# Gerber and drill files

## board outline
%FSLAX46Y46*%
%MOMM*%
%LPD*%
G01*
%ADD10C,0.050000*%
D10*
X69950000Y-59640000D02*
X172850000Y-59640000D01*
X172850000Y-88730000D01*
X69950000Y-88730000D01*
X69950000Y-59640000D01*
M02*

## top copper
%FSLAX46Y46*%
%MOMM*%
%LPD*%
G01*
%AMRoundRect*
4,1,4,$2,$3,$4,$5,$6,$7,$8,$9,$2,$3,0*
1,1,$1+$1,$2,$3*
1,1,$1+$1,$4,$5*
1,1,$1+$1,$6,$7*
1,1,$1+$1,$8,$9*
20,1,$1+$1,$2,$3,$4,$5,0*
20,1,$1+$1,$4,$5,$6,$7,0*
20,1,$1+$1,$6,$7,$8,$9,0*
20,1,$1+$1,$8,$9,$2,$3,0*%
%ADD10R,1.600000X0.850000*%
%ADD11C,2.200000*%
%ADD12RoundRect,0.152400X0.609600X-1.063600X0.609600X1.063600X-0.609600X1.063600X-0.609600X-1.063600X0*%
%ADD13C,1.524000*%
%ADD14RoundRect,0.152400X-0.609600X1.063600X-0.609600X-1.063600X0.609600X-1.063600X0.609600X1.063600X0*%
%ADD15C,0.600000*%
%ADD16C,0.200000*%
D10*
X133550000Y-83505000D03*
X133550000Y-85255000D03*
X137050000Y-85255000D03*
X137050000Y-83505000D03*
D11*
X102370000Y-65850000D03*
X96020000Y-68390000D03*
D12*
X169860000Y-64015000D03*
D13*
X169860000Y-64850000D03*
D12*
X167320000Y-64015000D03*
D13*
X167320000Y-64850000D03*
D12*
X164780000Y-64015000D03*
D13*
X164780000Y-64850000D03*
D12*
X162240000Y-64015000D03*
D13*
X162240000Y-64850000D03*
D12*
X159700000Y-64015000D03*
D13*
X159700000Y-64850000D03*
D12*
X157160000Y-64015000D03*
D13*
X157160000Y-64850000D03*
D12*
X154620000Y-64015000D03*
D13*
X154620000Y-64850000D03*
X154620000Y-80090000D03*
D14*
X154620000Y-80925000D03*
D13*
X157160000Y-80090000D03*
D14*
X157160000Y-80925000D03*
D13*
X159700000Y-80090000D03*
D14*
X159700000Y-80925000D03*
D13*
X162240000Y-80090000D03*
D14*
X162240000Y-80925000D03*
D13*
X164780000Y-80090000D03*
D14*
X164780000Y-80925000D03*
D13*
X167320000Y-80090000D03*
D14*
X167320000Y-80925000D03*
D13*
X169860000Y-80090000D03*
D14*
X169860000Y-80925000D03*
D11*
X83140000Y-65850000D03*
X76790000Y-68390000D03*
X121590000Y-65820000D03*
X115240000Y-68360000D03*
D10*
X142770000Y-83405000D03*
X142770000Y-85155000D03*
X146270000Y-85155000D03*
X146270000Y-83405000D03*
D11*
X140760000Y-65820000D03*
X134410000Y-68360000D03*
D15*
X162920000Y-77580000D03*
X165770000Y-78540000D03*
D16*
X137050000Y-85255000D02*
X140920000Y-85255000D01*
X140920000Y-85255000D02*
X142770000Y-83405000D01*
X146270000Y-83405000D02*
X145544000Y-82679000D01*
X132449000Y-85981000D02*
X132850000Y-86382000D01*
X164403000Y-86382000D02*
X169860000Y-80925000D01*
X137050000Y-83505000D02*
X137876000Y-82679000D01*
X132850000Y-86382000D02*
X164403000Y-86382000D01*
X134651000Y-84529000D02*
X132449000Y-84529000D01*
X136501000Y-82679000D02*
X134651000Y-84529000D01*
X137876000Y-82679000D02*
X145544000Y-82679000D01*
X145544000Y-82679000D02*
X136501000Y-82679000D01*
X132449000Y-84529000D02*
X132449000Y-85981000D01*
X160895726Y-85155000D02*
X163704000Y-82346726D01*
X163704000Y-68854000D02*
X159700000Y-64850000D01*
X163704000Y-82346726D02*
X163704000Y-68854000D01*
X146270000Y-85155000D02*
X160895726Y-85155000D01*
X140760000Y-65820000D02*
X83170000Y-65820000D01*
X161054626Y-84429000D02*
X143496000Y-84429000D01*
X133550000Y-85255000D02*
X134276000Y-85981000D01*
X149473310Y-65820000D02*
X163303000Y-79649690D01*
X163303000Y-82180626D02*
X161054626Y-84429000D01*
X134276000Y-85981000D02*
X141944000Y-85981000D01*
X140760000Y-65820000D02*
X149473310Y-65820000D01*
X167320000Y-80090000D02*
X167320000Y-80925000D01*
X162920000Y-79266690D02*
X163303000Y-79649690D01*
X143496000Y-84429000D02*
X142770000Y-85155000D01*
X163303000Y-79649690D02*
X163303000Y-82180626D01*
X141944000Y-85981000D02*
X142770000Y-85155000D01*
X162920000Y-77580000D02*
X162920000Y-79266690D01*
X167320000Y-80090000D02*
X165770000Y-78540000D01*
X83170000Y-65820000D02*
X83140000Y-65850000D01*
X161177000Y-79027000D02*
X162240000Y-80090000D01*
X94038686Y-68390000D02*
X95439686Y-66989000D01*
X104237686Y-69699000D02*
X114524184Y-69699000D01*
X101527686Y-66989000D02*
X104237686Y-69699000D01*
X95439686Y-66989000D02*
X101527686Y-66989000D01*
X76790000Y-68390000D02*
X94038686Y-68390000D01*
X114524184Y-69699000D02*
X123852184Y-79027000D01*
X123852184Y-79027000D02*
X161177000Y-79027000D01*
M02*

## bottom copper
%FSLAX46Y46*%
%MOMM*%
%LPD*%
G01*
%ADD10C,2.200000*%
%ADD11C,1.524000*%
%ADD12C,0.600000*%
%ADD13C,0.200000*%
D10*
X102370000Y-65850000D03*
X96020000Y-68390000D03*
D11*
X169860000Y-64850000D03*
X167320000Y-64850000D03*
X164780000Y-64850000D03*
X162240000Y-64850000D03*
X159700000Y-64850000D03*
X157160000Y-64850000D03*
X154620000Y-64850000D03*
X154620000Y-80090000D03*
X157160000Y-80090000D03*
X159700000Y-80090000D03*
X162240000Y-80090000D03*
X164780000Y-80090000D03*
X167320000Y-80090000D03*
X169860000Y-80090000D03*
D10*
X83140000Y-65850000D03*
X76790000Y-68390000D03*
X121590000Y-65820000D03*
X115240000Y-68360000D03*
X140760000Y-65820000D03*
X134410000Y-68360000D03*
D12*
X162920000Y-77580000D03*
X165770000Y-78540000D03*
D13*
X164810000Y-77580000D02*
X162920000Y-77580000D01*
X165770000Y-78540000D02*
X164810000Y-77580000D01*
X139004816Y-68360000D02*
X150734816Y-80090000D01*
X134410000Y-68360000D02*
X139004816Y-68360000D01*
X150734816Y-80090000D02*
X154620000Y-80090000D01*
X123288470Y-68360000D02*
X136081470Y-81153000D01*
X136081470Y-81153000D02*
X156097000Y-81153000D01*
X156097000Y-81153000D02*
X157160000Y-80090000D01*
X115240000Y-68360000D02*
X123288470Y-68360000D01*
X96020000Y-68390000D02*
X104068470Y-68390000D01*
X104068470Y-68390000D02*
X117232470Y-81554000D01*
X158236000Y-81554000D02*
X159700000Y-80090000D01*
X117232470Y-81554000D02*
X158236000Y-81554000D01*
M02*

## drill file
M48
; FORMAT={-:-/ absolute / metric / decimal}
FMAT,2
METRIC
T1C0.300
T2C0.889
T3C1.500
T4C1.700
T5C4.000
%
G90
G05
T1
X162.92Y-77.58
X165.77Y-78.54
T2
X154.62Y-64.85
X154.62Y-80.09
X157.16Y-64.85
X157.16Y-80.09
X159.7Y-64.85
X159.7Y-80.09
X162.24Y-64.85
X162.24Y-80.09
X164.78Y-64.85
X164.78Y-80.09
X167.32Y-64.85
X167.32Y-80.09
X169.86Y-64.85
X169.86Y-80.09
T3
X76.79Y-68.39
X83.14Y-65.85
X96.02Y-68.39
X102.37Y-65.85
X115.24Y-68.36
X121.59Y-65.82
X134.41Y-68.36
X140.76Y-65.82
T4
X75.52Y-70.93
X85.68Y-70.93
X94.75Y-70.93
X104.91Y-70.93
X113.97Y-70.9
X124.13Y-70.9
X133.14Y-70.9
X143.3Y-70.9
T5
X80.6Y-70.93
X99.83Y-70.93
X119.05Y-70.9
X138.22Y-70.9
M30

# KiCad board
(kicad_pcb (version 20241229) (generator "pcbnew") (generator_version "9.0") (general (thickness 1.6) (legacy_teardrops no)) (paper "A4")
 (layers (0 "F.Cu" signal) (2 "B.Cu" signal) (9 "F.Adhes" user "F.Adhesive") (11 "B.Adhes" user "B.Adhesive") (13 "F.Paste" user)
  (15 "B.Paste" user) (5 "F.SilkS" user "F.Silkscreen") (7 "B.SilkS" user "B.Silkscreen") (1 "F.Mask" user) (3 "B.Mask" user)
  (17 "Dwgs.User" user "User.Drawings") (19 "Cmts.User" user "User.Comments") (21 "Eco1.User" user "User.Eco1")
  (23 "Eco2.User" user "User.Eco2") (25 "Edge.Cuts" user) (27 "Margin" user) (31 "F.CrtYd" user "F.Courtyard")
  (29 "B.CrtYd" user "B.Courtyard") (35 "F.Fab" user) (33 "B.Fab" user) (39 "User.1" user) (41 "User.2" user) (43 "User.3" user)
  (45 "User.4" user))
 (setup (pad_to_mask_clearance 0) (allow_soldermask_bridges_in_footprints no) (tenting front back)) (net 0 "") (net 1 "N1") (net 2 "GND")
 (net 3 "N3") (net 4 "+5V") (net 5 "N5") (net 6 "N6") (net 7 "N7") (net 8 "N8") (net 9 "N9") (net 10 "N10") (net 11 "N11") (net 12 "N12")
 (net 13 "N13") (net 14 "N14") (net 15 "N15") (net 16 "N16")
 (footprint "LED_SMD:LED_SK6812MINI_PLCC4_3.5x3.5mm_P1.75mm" (layer "F.Cu") (at 135.3 84.38)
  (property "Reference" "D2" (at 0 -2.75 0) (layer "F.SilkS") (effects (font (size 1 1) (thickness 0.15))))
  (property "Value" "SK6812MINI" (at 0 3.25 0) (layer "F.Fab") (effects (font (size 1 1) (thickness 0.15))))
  (pad "1" smd rect (at -1.75 -0.875) (size 1.6 0.85) (layers "F.Cu" "F.Mask" "F.Paste") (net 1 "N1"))
  (pad "2" smd rect (at -1.75 0.875) (size 1.6 0.85) (layers "F.Cu" "F.Mask" "F.Paste") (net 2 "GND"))
  (pad "3" smd rect (at 1.75 0.875) (size 1.6 0.85) (layers "F.Cu" "F.Mask" "F.Paste") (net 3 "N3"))
  (pad "4" smd rect (at 1.75 -0.875) (size 1.6 0.85) (layers "F.Cu" "F.Mask" "F.Paste") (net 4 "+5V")))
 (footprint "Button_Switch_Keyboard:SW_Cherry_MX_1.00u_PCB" (layer "F.Cu") (at 102.37 65.85)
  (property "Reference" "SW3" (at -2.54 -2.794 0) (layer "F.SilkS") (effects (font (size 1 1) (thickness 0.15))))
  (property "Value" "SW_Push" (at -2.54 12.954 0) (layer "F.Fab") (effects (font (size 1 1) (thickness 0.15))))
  (pad "" np_thru_hole circle (at -7.62 5.08) (size 1.7 1.7) (drill 1.7) (layers "*.Cu" "*.Mask"))
  (pad "" np_thru_hole circle (at -2.54 5.08) (size 4 4) (drill 4) (layers "*.Cu" "*.Mask"))
  (pad "" np_thru_hole circle (at 2.54 5.08) (size 1.7 1.7) (drill 1.7) (layers "*.Cu" "*.Mask"))
  (pad "1" thru_hole circle (at 0 0) (size 2.2 2.2) (drill 1.5) (layers "*.Cu" "*.Mask") (remove_unused_layers no) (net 2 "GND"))
  (pad "2" thru_hole circle (at -6.35 2.54) (size 2.2 2.2) (drill 1.5) (layers "*.Cu" "*.Mask") (remove_unused_layers no) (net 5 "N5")))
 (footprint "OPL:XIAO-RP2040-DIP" (layer "F.Cu") (at 162.24 72.47 -90)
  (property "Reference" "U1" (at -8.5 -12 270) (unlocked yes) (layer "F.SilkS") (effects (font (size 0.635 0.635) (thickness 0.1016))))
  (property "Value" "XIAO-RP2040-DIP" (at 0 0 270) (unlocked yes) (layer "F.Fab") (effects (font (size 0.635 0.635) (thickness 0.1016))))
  (pad "1" smd roundrect (at -8.455 -7.62 90) (size 2.432 1.524) (layers "F.Cu" "F.Mask") (roundrect_rratio 0.1) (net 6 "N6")
   (thermal_bridge_angle 45))
  (pad "1" thru_hole circle (at -7.62 -7.62 90) (size 1.524 1.524) (drill 0.889) (layers "*.Cu" "*.Mask") (remove_unused_layers no)
   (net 6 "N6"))
  (pad "2" smd roundrect (at -8.455 -5.08 90) (size 2.432 1.524) (layers "F.Cu" "F.Mask") (roundrect_rratio 0.1) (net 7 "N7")
   (thermal_bridge_angle 45))
  (pad "2" thru_hole circle (at -7.62 -5.08 90) (size 1.524 1.524) (drill 0.889) (layers "*.Cu" "*.Mask") (remove_unused_layers no)
   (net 7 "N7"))
  (pad "3" smd roundrect (at -8.455 -2.54 90) (size 2.432 1.524) (layers "F.Cu" "F.Mask") (roundrect_rratio 0.1) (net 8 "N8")
   (thermal_bridge_angle 45))
  (pad "3" thru_hole circle (at -7.62 -2.54 90) (size 1.524 1.524) (drill 0.889) (layers "*.Cu" "*.Mask") (remove_unused_layers no)
   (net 8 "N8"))
  (pad "4" smd roundrect (at -8.455 0 90) (size 2.432 1.524) (layers "F.Cu" "F.Mask") (roundrect_rratio 0.1) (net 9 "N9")
   (thermal_bridge_angle 45))
  (pad "4" thru_hole circle (at -7.62 0 90) (size 1.524 1.524) (drill 0.889) (layers "*.Cu" "*.Mask") (remove_unused_layers no) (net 9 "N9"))
  (pad "5" smd roundrect (at -8.455 2.54 90) (size 2.432 1.524) (layers "F.Cu" "F.Mask") (roundrect_rratio 0.1) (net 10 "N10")
   (thermal_bridge_angle 45))
  (pad "5" thru_hole circle (at -7.62 2.54 90) (size 1.524 1.524) (drill 0.889) (layers "*.Cu" "*.Mask") (remove_unused_layers no)
   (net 10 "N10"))
  (pad "6" smd roundrect (at -8.455 5.08 90) (size 2.432 1.524) (layers "F.Cu" "F.Mask") (roundrect_rratio 0.1) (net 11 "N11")
   (thermal_bridge_angle 45))
  (pad "6" thru_hole circle (at -7.62 5.08 90) (size 1.524 1.524) (drill 0.889) (layers "*.Cu" "*.Mask") (remove_unused_layers no)
   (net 11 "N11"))
  (pad "7" smd roundrect (at -8.455 7.62 90) (size 2.432 1.524) (layers "F.Cu" "F.Mask") (roundrect_rratio 0.1) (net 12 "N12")
   (thermal_bridge_angle 45))
  (pad "7" thru_hole circle (at -7.62 7.62 90) (size 1.524 1.524) (drill 0.889) (layers "*.Cu" "*.Mask") (remove_unused_layers no)
   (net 12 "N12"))
  (pad "8" thru_hole circle (at 7.62 7.62 270) (size 1.524 1.524) (drill 0.889) (layers "*.Cu" "*.Mask") (remove_unused_layers no)
   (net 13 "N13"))
  (pad "8" smd roundrect (at 8.455 7.62 270) (size 2.432 1.524) (layers "F.Cu" "F.Mask") (roundrect_rratio 0.1) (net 13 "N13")
   (thermal_bridge_angle 45))
  (pad "9" thru_hole circle (at 7.62 5.08 270) (size 1.524 1.524) (drill 0.889) (layers "*.Cu" "*.Mask") (remove_unused_layers no)
   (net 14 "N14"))
  (pad "9" smd roundrect (at 8.455 5.08 270) (size 2.432 1.524) (layers "F.Cu" "F.Mask") (roundrect_rratio 0.1) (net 14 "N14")
   (thermal_bridge_angle 45))
  (pad "10" thru_hole circle (at 7.62 2.54 270) (size 1.524 1.524) (drill 0.889) (layers "*.Cu" "*.Mask") (remove_unused_layers no)
   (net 5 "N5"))
  (pad "10" smd roundrect (at 8.455 2.54 270) (size 2.432 1.524) (layers "F.Cu" "F.Mask") (roundrect_rratio 0.1) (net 5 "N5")
   (thermal_bridge_angle 45))
  (pad "11" thru_hole circle (at 7.62 0 270) (size 1.524 1.524) (drill 0.889) (layers "*.Cu" "*.Mask") (remove_unused_layers no)
   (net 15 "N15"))
  (pad "11" smd roundrect (at 8.455 0 270) (size 2.432 1.524) (layers "F.Cu" "F.Mask") (roundrect_rratio 0.1) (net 15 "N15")
   (thermal_bridge_angle 45))
  (pad "12" thru_hole circle (at 7.62 -2.54 270) (size 1.524 1.524) (drill 0.889) (layers "*.Cu" "*.Mask") (remove_unused_layers no)
   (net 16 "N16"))
  (pad "12" smd roundrect (at 8.455 -2.54 270) (size 2.432 1.524) (layers "F.Cu" "F.Mask") (roundrect_rratio 0.1) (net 16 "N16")
   (thermal_bridge_angle 45))
  (pad "13" thru_hole circle (at 7.62 -5.08 270) (size 1.524 1.524) (drill 0.889) (layers "*.Cu" "*.Mask") (remove_unused_layers no)
   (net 2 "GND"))
  (pad "13" smd roundrect (at 8.455 -5.08 270) (size 2.432 1.524) (layers "F.Cu" "F.Mask") (roundrect_rratio 0.1) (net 2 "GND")
   (thermal_bridge_angle 45))
  (pad "14" thru_hole circle (at 7.62 -7.62 270) (size 1.524 1.524) (drill 0.889) (layers "*.Cu" "*.Mask") (remove_unused_layers no)
   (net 4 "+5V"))
  (pad "14" smd roundrect (at 8.455 -7.62 270) (size 2.432 1.524) (layers "F.Cu" "F.Mask") (roundrect_rratio 0.1) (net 4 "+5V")
   (thermal_bridge_angle 45)))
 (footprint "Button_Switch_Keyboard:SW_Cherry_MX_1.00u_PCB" (layer "F.Cu") (at 83.14 65.85)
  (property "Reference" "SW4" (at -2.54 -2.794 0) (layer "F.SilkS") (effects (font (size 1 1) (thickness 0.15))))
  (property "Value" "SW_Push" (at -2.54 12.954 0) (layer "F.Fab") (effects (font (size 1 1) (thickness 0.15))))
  (pad "" np_thru_hole circle (at -7.62 5.08) (size 1.7 1.7) (drill 1.7) (layers "*.Cu" "*.Mask"))
  (pad "" np_thru_hole circle (at -2.54 5.08) (size 4 4) (drill 4) (layers "*.Cu" "*.Mask"))
  (pad "" np_thru_hole circle (at 2.54 5.08) (size 1.7 1.7) (drill 1.7) (layers "*.Cu" "*.Mask"))
  (pad "1" thru_hole circle (at 0 0) (size 2.2 2.2) (drill 1.5) (layers "*.Cu" "*.Mask") (remove_unused_layers no) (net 2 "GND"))
  (pad "2" thru_hole circle (at -6.35 2.54) (size 2.2 2.2) (drill 1.5) (layers "*.Cu" "*.Mask") (remove_unused_layers no) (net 15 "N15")))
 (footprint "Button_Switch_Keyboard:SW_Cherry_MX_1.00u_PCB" (layer "F.Cu") (at 121.59 65.82)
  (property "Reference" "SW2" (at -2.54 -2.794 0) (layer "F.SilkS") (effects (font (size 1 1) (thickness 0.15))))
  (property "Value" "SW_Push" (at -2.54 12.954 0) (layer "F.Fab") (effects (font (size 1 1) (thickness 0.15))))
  (pad "" np_thru_hole circle (at -7.62 5.08) (size 1.7 1.7) (drill 1.7) (layers "*.Cu" "*.Mask"))
  (pad "" np_thru_hole circle (at -2.54 5.08) (size 4 4) (drill 4) (layers "*.Cu" "*.Mask"))
  (pad "" np_thru_hole circle (at 2.54 5.08) (size 1.7 1.7) (drill 1.7) (layers "*.Cu" "*.Mask"))
  (pad "1" thru_hole circle (at 0 0) (size 2.2 2.2) (drill 1.5) (layers "*.Cu" "*.Mask") (remove_unused_layers no) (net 2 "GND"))
  (pad "2" thru_hole circle (at -6.35 2.54) (size 2.2 2.2) (drill 1.5) (layers "*.Cu" "*.Mask") (remove_unused_layers no) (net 14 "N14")))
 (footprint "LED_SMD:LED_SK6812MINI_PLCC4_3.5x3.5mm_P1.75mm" (layer "F.Cu") (at 144.52 84.28)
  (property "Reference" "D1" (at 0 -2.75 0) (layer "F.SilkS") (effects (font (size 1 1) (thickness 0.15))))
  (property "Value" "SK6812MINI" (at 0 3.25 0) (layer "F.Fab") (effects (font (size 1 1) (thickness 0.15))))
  (pad "1" smd rect (at -1.75 -0.875) (size 1.6 0.85) (layers "F.Cu" "F.Mask" "F.Paste") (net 3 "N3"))
  (pad "2" smd rect (at -1.75 0.875) (size 1.6 0.85) (layers "F.Cu" "F.Mask" "F.Paste") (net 2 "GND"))
  (pad "3" smd rect (at 1.75 0.875) (size 1.6 0.85) (layers "F.Cu" "F.Mask" "F.Paste") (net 10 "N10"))
  (pad "4" smd rect (at 1.75 -0.875) (size 1.6 0.85) (layers "F.Cu" "F.Mask" "F.Paste") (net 4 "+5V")))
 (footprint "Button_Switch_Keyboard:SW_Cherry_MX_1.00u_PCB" (layer "F.Cu") (at 140.76 65.82)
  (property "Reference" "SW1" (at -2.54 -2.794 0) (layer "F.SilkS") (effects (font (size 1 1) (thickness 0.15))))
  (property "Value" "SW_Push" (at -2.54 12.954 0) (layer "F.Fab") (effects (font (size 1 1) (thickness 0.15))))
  (pad "" np_thru_hole circle (at -7.62 5.08) (size 1.7 1.7) (drill 1.7) (layers "*.Cu" "*.Mask"))
  (pad "" np_thru_hole circle (at -2.54 5.08) (size 4 4) (drill 4) (layers "*.Cu" "*.Mask"))
  (pad "" np_thru_hole circle (at 2.54 5.08) (size 1.7 1.7) (drill 1.7) (layers "*.Cu" "*.Mask"))
  (pad "1" thru_hole circle (at 0 0) (size 2.2 2.2) (drill 1.5) (layers "*.Cu" "*.Mask") (remove_unused_layers no) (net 2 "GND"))
  (pad "2" thru_hole circle (at -6.35 2.54) (size 2.2 2.2) (drill 1.5) (layers "*.Cu" "*.Mask") (remove_unused_layers no) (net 13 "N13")))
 (gr_rect (start 69.95 59.64) (end 172.85 88.73) (stroke (width 0.05) (type default)) (fill no) (layer "Edge.Cuts"))
 (segment (start 137.05 85.255) (end 140.92 85.255) (width 0.2) (layer "F.Cu") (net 3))
 (segment (start 140.92 85.255) (end 142.77 83.405) (width 0.2) (layer "F.Cu") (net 3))
 (segment (start 146.27 83.405) (end 145.544 82.679) (width 0.2) (layer "F.Cu") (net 4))
 (segment (start 132.449 85.981) (end 132.85 86.382) (width 0.2) (layer "F.Cu") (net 4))
 (segment (start 164.403 86.382) (end 169.86 80.925) (width 0.2) (layer "F.Cu") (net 4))
 (segment (start 137.05 83.505) (end 137.876 82.679) (width 0.2) (layer "F.Cu") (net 4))
 (segment (start 132.85 86.382) (end 164.403 86.382) (width 0.2) (layer "F.Cu") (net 4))
 (segment (start 134.651 84.529) (end 132.449 84.529) (width 0.2) (layer "F.Cu") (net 4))
 (segment (start 136.501 82.679) (end 134.651 84.529) (width 0.2) (layer "F.Cu") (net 4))
 (segment (start 137.876 82.679) (end 145.544 82.679) (width 0.2) (layer "F.Cu") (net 4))
 (segment (start 145.544 82.679) (end 136.501 82.679) (width 0.2) (layer "F.Cu") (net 4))
 (segment (start 132.449 84.529) (end 132.449 85.981) (width 0.2) (layer "F.Cu") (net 4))
 (segment (start 160.895726 85.155) (end 163.704 82.346726) (width 0.2) (layer "F.Cu") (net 10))
 (segment (start 163.704 68.854) (end 159.7 64.85) (width 0.2) (layer "F.Cu") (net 10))
 (segment (start 163.704 82.346726) (end 163.704 68.854) (width 0.2) (layer "F.Cu") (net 10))
 (segment (start 146.27 85.155) (end 160.895726 85.155) (width 0.2) (layer "F.Cu") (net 10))
 (segment (start 140.76 65.82) (end 83.17 65.82) (width 0.2) (layer "F.Cu") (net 2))
 (segment (start 161.054626 84.429) (end 143.496 84.429) (width 0.2) (layer "F.Cu") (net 2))
 (segment (start 133.55 85.255) (end 134.276 85.981) (width 0.2) (layer "F.Cu") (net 2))
 (segment (start 149.47331 65.82) (end 163.303 79.64969) (width 0.2) (layer "F.Cu") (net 2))
 (segment (start 163.303 82.180626) (end 161.054626 84.429) (width 0.2) (layer "F.Cu") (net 2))
 (segment (start 134.276 85.981) (end 141.944 85.981) (width 0.2) (layer "F.Cu") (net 2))
 (segment (start 140.76 65.82) (end 149.47331 65.82) (width 0.2) (layer "F.Cu") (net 2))
 (segment (start 167.32 80.09) (end 167.32 80.925) (width 0.2) (layer "F.Cu") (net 2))
 (segment (start 162.92 79.26669) (end 163.303 79.64969) (width 0.2) (layer "F.Cu") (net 2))
 (segment (start 143.496 84.429) (end 142.77 85.155) (width 0.2) (layer "F.Cu") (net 2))
 (segment (start 163.303 79.64969) (end 163.303 82.180626) (width 0.2) (layer "F.Cu") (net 2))
 (segment (start 141.944 85.981) (end 142.77 85.155) (width 0.2) (layer "F.Cu") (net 2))
 (segment (start 162.92 77.58) (end 162.92 79.26669) (width 0.2) (layer "F.Cu") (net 2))
 (segment (start 167.32 80.09) (end 165.77 78.54) (width 0.2) (layer "F.Cu") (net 2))
 (segment (start 83.17 65.82) (end 83.14 65.85) (width 0.2) (layer "F.Cu") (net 2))
 (via (at 162.92 77.58) (size 0.6) (drill 0.3) (layers "F.Cu" "B.Cu") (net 2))
 (via (at 165.77 78.54) (size 0.6) (drill 0.3) (layers "F.Cu" "B.Cu") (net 2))
 (segment (start 164.81 77.58) (end 162.92 77.58) (width 0.2) (layer "B.Cu") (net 2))
 (segment (start 165.77 78.54) (end 164.81 77.58) (width 0.2) (layer "B.Cu") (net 2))
 (segment (start 139.004816 68.36) (end 150.734816 80.09) (width 0.2) (layer "B.Cu") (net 13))
 (segment (start 134.41 68.36) (end 139.004816 68.36) (width 0.2) (layer "B.Cu") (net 13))
 (segment (start 150.734816 80.09) (end 154.62 80.09) (width 0.2) (layer "B.Cu") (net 13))
 (segment (start 123.28847 68.36) (end 136.08147 81.153) (width 0.2) (layer "B.Cu") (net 14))
 (segment (start 136.08147 81.153) (end 156.097 81.153) (width 0.2) (layer "B.Cu") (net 14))
 (segment (start 156.097 81.153) (end 157.16 80.09) (width 0.2) (layer "B.Cu") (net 14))
 (segment (start 115.24 68.36) (end 123.28847 68.36) (width 0.2) (layer "B.Cu") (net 14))
 (segment (start 96.02 68.39) (end 104.06847 68.39) (width 0.2) (layer "B.Cu") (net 5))
 (segment (start 104.06847 68.39) (end 117.23247 81.554) (width 0.2) (layer "B.Cu") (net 5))
 (segment (start 158.236 81.554) (end 159.7 80.09) (width 0.2) (layer "B.Cu") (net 5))
 (segment (start 117.23247 81.554) (end 158.236 81.554) (width 0.2) (layer "B.Cu") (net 5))
 (segment (start 161.177 79.027) (end 162.24 80.09) (width 0.2) (layer "F.Cu") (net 15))
 (segment (start 94.038686 68.39) (end 95.439686 66.989) (width 0.2) (layer "F.Cu") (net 15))
 (segment (start 104.237686 69.699) (end 114.524184 69.699) (width 0.2) (layer "F.Cu") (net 15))
 (segment (start 101.527686 66.989) (end 104.237686 69.699) (width 0.2) (layer "F.Cu") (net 15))
 (segment (start 95.439686 66.989) (end 101.527686 66.989) (width 0.2) (layer "F.Cu") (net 15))
 (segment (start 76.79 68.39) (end 94.038686 68.39) (width 0.2) (layer "F.Cu") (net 15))
 (segment (start 114.524184 69.699) (end 123.852184 79.027) (width 0.2) (layer "F.Cu") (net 15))
 (segment (start 123.852184 79.027) (end 161.177 79.027) (width 0.2) (layer "F.Cu") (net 15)))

